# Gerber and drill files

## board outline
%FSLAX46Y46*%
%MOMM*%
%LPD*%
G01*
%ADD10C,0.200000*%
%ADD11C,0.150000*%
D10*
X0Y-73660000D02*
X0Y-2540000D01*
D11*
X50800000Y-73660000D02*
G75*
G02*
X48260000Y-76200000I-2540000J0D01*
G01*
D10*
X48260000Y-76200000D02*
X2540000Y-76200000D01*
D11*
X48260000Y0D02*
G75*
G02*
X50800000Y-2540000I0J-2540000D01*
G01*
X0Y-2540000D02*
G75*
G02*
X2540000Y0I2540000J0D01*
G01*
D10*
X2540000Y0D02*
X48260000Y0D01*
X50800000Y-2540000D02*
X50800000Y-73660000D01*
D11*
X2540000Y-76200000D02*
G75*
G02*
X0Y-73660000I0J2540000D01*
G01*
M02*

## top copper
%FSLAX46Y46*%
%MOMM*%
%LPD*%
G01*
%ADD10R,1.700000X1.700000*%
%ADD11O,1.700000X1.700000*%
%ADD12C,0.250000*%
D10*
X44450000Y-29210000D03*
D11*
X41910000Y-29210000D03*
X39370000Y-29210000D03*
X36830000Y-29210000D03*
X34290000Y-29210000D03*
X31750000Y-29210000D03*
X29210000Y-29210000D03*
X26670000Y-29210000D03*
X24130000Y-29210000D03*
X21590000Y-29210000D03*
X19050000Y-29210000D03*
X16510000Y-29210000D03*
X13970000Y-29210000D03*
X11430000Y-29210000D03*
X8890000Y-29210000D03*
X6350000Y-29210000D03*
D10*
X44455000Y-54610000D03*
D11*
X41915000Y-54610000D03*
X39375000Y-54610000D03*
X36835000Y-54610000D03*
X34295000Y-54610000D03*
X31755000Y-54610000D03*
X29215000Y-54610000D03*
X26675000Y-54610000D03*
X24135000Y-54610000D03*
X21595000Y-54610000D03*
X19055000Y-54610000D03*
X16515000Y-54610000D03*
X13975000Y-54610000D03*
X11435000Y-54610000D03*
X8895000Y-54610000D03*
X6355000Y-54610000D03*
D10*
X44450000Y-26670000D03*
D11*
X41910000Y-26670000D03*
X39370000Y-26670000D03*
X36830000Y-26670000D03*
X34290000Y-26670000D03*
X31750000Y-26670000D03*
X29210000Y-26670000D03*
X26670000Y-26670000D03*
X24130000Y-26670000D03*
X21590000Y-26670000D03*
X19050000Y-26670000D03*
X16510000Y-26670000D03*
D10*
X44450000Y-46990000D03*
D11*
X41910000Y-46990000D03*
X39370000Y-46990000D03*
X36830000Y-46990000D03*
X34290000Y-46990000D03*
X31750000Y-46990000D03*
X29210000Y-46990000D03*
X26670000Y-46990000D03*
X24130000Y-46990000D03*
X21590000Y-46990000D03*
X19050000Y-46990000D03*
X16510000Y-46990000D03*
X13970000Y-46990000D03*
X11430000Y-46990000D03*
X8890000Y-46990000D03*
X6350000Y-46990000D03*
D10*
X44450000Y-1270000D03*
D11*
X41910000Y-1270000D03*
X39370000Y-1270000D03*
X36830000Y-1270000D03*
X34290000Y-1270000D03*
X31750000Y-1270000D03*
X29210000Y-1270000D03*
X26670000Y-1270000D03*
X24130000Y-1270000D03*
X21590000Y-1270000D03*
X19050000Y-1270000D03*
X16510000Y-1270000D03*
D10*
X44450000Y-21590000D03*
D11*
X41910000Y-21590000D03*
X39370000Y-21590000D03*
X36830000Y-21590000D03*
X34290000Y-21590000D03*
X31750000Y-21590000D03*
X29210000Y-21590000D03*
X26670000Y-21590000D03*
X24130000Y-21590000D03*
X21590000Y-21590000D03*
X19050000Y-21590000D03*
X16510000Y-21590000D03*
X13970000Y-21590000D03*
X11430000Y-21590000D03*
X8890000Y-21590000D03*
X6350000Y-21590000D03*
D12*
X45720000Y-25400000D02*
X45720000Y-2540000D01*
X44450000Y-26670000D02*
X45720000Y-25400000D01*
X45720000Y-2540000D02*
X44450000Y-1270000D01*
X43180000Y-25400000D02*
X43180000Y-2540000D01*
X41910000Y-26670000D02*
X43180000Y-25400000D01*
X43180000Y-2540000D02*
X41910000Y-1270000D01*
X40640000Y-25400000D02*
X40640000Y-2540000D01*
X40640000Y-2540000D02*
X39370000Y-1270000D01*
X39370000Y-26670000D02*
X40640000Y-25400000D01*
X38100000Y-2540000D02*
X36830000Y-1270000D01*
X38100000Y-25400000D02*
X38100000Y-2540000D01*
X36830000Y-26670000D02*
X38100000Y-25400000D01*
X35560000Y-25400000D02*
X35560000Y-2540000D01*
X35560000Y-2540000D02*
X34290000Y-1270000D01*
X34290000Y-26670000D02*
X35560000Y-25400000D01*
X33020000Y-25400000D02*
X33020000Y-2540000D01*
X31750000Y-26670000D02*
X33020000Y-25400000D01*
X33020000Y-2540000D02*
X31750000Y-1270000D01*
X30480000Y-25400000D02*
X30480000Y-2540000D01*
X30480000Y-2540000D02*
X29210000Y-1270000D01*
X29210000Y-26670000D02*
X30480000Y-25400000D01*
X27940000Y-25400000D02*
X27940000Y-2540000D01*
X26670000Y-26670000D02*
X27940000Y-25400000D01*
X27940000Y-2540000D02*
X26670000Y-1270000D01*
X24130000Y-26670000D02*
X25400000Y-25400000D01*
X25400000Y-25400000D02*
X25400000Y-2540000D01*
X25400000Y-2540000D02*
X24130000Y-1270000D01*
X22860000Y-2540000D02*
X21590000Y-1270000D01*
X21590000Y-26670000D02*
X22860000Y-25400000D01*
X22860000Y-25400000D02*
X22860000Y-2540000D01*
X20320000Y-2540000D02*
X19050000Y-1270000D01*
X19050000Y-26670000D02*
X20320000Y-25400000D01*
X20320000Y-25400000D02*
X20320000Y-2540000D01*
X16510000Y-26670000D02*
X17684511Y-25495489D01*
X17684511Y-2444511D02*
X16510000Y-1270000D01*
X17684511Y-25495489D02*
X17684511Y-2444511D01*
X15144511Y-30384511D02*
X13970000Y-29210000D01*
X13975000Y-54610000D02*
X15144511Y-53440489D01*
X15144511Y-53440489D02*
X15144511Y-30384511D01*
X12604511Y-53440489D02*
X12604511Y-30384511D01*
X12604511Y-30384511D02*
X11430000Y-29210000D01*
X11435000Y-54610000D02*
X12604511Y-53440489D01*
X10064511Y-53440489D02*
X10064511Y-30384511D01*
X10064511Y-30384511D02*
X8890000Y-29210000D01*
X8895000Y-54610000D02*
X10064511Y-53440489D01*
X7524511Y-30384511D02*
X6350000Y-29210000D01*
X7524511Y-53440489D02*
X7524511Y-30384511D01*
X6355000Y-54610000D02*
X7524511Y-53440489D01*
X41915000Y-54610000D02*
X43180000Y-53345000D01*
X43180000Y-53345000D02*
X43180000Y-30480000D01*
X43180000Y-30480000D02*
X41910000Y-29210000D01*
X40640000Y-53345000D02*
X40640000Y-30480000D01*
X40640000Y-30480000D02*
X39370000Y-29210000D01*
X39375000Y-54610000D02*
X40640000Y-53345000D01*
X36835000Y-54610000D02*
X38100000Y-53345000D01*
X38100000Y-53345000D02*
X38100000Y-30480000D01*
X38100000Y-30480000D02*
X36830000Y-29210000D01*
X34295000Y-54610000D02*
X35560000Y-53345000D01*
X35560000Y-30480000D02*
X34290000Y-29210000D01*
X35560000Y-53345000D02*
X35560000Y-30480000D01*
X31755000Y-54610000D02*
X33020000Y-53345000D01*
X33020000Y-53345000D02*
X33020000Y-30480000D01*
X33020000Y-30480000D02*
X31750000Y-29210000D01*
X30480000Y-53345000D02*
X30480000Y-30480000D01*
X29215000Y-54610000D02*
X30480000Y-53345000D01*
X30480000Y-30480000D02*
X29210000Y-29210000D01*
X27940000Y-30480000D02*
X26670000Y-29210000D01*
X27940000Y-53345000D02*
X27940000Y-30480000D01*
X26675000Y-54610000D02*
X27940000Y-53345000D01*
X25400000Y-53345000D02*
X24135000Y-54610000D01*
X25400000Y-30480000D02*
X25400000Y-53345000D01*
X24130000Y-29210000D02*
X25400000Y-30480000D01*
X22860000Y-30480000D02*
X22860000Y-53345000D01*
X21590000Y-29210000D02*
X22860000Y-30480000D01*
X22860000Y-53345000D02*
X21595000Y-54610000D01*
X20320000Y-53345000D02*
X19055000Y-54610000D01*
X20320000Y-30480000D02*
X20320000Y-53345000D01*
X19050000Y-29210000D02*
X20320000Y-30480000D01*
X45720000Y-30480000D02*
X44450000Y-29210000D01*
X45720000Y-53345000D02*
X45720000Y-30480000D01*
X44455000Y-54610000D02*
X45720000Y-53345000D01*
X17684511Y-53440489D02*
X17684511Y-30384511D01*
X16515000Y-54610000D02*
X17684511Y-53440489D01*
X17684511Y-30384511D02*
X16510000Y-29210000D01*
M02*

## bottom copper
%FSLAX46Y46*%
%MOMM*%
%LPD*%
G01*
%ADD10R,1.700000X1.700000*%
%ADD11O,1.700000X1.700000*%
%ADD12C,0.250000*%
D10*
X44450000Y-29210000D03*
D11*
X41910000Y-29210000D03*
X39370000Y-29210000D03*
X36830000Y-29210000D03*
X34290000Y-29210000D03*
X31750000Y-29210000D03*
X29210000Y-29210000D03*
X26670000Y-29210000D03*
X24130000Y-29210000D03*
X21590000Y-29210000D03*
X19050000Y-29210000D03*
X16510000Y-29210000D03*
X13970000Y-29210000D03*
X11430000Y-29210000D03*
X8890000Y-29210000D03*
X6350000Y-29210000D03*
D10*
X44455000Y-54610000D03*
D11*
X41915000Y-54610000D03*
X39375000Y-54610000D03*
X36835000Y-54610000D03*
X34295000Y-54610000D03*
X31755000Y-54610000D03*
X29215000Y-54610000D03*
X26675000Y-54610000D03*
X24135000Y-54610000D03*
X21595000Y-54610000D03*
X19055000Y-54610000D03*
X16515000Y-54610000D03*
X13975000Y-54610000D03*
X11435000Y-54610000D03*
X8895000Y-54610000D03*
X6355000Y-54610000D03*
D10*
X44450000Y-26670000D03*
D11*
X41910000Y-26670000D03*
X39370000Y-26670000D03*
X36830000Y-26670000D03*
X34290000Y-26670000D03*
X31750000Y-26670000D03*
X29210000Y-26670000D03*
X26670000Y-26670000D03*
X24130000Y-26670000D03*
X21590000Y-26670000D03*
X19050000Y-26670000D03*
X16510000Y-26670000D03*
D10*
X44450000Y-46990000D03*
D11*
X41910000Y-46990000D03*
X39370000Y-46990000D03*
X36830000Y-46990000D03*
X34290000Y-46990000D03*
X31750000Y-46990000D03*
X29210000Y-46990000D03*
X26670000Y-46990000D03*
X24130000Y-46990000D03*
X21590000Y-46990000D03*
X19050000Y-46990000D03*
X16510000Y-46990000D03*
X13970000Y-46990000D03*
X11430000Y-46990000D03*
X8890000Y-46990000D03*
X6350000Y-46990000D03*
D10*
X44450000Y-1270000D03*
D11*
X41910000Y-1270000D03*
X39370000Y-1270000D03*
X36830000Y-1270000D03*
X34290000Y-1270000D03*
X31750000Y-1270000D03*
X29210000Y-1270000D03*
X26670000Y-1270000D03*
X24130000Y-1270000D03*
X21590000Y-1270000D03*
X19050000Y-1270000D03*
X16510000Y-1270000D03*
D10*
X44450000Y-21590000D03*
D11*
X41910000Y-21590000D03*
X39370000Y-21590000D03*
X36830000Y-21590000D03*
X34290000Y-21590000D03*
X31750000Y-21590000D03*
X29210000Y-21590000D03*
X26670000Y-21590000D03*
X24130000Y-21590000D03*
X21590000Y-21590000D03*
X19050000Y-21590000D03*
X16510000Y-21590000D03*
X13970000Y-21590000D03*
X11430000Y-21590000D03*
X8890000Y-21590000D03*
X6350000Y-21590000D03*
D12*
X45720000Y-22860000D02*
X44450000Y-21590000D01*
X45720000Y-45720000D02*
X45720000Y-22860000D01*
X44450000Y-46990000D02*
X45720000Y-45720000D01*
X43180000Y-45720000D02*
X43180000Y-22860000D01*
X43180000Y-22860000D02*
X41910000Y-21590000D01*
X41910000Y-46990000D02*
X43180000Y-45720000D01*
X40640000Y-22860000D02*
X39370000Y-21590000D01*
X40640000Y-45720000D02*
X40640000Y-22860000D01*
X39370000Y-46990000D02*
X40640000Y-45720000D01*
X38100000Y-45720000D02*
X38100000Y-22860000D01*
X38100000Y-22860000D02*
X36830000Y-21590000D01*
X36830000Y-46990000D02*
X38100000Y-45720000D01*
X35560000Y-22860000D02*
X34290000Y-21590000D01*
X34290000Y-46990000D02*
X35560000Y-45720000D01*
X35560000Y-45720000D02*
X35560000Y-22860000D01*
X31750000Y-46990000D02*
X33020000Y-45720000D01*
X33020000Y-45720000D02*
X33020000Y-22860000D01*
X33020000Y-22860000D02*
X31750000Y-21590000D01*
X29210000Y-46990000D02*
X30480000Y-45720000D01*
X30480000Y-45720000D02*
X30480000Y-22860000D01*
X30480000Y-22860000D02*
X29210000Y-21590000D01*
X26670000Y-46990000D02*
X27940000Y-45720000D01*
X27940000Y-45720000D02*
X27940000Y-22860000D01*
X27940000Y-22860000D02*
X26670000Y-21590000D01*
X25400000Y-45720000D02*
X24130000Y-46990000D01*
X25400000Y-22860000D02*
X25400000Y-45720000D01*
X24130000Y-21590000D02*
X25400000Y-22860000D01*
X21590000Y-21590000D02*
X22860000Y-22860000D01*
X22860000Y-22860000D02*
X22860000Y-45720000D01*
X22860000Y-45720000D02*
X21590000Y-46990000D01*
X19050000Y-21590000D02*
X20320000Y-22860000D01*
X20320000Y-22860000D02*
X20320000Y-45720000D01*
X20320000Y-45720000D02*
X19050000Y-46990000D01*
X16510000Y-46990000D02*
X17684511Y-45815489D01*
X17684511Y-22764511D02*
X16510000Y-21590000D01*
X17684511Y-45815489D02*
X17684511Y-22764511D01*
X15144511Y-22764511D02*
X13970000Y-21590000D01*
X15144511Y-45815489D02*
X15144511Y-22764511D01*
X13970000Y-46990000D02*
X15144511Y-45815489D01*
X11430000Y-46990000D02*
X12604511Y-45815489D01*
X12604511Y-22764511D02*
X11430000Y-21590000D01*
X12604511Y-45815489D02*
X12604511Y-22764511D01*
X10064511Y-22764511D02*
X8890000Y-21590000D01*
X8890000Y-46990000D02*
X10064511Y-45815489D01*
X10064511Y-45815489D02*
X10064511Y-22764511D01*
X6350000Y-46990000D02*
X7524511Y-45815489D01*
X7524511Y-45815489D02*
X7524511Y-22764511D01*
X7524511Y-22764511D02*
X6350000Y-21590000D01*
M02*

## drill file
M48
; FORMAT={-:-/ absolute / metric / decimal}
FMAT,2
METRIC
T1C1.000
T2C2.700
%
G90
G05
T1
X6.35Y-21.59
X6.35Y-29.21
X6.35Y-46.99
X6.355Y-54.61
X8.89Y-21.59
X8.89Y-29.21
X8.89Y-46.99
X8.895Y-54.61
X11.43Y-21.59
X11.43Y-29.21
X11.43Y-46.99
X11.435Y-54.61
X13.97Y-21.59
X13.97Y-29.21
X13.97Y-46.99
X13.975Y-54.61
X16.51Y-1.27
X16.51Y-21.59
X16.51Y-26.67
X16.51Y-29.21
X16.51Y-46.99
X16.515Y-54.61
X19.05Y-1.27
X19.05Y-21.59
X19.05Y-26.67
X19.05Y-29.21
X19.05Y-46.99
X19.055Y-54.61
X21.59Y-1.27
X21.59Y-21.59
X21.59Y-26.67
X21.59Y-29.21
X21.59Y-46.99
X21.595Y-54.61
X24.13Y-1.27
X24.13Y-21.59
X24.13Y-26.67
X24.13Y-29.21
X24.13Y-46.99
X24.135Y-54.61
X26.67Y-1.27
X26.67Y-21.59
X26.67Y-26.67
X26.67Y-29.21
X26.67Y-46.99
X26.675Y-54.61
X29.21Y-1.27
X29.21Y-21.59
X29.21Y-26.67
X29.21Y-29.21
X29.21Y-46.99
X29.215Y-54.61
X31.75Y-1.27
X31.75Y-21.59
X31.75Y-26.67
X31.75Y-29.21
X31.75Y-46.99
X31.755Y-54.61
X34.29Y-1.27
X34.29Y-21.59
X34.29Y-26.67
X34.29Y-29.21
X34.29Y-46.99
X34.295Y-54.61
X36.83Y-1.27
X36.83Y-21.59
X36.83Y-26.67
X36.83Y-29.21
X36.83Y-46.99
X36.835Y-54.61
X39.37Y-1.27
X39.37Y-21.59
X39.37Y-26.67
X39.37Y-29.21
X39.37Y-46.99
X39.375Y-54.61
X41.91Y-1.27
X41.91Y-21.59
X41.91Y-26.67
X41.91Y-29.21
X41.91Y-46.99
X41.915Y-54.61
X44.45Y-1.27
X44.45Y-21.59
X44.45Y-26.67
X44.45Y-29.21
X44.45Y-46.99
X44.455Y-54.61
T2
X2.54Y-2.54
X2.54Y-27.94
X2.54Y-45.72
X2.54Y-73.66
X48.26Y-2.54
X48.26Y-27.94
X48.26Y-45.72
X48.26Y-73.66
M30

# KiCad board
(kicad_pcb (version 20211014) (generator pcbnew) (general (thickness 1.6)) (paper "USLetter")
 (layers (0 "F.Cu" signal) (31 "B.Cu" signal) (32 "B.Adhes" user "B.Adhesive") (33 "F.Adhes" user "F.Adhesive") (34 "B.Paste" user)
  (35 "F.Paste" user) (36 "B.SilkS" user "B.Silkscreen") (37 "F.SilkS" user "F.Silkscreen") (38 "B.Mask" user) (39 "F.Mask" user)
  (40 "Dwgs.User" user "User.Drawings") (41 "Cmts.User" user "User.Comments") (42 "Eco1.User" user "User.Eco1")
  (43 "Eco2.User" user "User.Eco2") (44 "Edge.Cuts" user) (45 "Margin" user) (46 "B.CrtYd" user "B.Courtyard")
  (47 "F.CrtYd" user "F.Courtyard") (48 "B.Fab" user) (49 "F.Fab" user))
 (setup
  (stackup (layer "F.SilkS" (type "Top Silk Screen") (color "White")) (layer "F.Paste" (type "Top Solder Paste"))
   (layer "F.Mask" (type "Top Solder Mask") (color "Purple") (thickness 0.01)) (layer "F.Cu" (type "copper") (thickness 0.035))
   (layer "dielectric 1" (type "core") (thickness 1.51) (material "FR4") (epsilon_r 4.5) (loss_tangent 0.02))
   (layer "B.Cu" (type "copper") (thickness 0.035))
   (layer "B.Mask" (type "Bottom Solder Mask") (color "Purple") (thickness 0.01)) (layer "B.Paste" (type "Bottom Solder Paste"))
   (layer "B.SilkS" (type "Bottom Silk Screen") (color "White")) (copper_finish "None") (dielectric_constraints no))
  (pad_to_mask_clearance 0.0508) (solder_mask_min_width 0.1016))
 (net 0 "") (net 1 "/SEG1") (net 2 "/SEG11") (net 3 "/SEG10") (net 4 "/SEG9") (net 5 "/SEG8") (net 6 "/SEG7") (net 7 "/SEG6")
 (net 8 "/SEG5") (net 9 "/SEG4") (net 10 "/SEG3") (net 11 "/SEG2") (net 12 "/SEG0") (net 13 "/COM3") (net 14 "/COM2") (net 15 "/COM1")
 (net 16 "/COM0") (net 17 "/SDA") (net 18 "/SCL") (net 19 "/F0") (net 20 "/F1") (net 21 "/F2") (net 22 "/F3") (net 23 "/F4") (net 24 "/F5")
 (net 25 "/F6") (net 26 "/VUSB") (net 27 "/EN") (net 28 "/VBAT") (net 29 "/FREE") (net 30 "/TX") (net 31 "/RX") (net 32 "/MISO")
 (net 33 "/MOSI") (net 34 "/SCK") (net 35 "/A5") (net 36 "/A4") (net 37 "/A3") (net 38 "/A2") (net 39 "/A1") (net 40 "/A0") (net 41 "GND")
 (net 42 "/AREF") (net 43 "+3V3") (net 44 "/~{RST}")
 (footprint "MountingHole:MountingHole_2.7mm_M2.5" (layer "F.Cu") (at 48.26 2.54)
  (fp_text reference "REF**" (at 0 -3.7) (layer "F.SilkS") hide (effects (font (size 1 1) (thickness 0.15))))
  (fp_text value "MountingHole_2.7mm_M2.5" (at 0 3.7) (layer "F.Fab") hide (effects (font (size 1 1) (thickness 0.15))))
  (pad "" np_thru_hole circle locked (at 0 0) (size 2.7 2.7) (drill 2.7) (layers *.Cu *.Mask)))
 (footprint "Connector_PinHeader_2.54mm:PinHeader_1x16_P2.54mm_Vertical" (layer "F.Cu") (at 44.45 29.21 -90)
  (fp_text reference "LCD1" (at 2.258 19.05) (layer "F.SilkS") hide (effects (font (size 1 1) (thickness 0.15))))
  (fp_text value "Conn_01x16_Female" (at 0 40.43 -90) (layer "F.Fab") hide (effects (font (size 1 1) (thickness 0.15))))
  (pad "1" thru_hole rect (at 0 0 270) (size 1.7 1.7) (drill 1) (layers *.Cu *.Mask) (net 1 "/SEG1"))
  (pad "2" thru_hole oval (at 0 2.54 270) (size 1.7 1.7) (drill 1) (layers *.Cu *.Mask) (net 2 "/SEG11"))
  (pad "3" thru_hole oval (at 0 5.08 270) (size 1.7 1.7) (drill 1) (layers *.Cu *.Mask) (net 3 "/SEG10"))
  (pad "4" thru_hole oval (at 0 7.62 270) (size 1.7 1.7) (drill 1) (layers *.Cu *.Mask) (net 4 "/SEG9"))
  (pad "5" thru_hole oval (at 0 10.16 270) (size 1.7 1.7) (drill 1) (layers *.Cu *.Mask) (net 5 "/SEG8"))
  (pad "6" thru_hole oval (at 0 12.7 270) (size 1.7 1.7) (drill 1) (layers *.Cu *.Mask) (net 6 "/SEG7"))
  (pad "7" thru_hole oval (at 0 15.24 270) (size 1.7 1.7) (drill 1) (layers *.Cu *.Mask) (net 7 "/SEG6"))
  (pad "8" thru_hole oval (at 0 17.78 270) (size 1.7 1.7) (drill 1) (layers *.Cu *.Mask) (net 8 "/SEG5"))
  (pad "9" thru_hole oval (at 0 20.32 270) (size 1.7 1.7) (drill 1) (layers *.Cu *.Mask) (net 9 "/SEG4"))
  (pad "10" thru_hole oval (at 0 22.86 270) (size 1.7 1.7) (drill 1) (layers *.Cu *.Mask) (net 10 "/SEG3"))
  (pad "11" thru_hole oval (at 0 25.4 270) (size 1.7 1.7) (drill 1) (layers *.Cu *.Mask) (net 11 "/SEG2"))
  (pad "12" thru_hole oval (at 0 27.94 270) (size 1.7 1.7) (drill 1) (layers *.Cu *.Mask) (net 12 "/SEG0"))
  (pad "13" thru_hole oval (at 0 30.48 270) (size 1.7 1.7) (drill 1) (layers *.Cu *.Mask) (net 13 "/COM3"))
  (pad "14" thru_hole oval (at 0 33.02 270) (size 1.7 1.7) (drill 1) (layers *.Cu *.Mask) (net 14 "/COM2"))
  (pad "15" thru_hole oval (at 0 35.56 270) (size 1.7 1.7) (drill 1) (layers *.Cu *.Mask) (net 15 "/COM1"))
  (pad "16" thru_hole oval (at 0 38.1 270) (size 1.7 1.7) (drill 1) (layers *.Cu *.Mask) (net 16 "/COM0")))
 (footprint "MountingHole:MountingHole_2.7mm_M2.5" (layer "F.Cu") (at 2.54 27.94)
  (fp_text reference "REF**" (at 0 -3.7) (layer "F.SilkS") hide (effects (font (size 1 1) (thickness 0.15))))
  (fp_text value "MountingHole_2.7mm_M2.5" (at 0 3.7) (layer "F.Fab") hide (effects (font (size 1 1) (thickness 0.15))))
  (pad "" np_thru_hole circle locked (at 0 0) (size 2.7 2.7) (drill 2.7) (layers *.Cu *.Mask)))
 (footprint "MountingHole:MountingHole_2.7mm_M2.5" (layer "F.Cu") (at 2.54 73.66)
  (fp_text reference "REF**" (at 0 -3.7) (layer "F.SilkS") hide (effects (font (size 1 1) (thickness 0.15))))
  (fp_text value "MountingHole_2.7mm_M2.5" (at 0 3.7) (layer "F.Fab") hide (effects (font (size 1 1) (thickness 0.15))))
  (pad "" np_thru_hole circle locked (at 0 0) (size 2.7 2.7) (drill 2.7) (layers *.Cu *.Mask)))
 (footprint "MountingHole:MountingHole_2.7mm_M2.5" (layer "F.Cu") (at 2.54 45.72)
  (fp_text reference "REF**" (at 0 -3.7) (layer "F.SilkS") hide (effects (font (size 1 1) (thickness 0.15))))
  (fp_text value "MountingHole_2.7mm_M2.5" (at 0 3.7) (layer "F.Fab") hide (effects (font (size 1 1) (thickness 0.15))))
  (pad "" np_thru_hole circle locked (at 0 0) (size 2.7 2.7) (drill 2.7) (layers *.Cu *.Mask)))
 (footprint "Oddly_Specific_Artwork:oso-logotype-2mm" (layer "F.Cu") (at 25.4 70.866)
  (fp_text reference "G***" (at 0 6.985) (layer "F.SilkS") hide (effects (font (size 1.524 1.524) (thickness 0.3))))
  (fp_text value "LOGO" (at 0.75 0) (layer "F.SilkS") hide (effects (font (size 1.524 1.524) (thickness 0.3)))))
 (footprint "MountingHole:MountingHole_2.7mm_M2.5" (layer "F.Cu") (at 48.26 45.72)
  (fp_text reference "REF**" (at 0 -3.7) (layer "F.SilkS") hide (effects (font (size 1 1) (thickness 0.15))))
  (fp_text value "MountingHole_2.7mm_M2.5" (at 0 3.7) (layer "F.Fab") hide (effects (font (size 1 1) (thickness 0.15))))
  (pad "" np_thru_hole circle locked (at 0 0) (size 2.7 2.7) (drill 2.7) (layers *.Cu *.Mask)))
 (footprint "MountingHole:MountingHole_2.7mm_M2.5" (layer "F.Cu") (at 48.26 73.66)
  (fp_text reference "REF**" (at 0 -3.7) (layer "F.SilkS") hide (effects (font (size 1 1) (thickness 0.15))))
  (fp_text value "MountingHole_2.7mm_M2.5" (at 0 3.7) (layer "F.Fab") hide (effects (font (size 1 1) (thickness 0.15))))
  (pad "" np_thru_hole circle locked (at 0 0) (size 2.7 2.7) (drill 2.7) (layers *.Cu *.Mask)))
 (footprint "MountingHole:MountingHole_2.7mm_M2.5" (layer "F.Cu") (at 2.54 2.54)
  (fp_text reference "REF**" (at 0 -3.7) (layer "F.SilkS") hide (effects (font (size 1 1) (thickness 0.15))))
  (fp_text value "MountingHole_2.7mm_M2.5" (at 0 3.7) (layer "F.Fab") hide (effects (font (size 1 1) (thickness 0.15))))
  (pad "" np_thru_hole circle locked (at 0 0) (size 2.7 2.7) (drill 2.7) (layers *.Cu *.Mask)))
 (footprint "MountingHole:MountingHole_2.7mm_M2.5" (layer "F.Cu") (at 48.26 27.94)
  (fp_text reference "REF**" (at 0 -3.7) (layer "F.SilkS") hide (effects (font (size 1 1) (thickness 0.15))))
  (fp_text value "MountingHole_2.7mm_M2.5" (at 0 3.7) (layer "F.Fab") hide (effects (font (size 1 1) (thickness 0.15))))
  (pad "" np_thru_hole circle locked (at 0 0) (size 2.7 2.7) (drill 2.7) (layers *.Cu *.Mask)))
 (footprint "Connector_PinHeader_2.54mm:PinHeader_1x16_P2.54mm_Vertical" (layer "F.Cu") (at 44.455 54.61 -90)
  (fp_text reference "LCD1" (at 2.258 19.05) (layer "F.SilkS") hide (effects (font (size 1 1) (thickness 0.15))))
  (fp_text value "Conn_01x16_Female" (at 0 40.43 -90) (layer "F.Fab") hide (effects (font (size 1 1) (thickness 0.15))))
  (pad "1" thru_hole rect (at 0 0 270) (size 1.7 1.7) (drill 1) (layers *.Cu *.Mask) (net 1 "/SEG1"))
  (pad "2" thru_hole oval (at 0 2.54 270) (size 1.7 1.7) (drill 1) (layers *.Cu *.Mask) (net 2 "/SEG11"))
  (pad "3" thru_hole oval (at 0 5.08 270) (size 1.7 1.7) (drill 1) (layers *.Cu *.Mask) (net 3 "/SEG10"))
  (pad "4" thru_hole oval (at 0 7.62 270) (size 1.7 1.7) (drill 1) (layers *.Cu *.Mask) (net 4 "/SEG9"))
  (pad "5" thru_hole oval (at 0 10.16 270) (size 1.7 1.7) (drill 1) (layers *.Cu *.Mask) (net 5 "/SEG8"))
  (pad "6" thru_hole oval (at 0 12.7 270) (size 1.7 1.7) (drill 1) (layers *.Cu *.Mask) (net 6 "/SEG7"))
  (pad "7" thru_hole oval (at 0 15.24 270) (size 1.7 1.7) (drill 1) (layers *.Cu *.Mask) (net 7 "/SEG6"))
  (pad "8" thru_hole oval (at 0 17.78 270) (size 1.7 1.7) (drill 1) (layers *.Cu *.Mask) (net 8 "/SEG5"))
  (pad "9" thru_hole oval (at 0 20.32 270) (size 1.7 1.7) (drill 1) (layers *.Cu *.Mask) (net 9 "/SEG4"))
  (pad "10" thru_hole oval (at 0 22.86 270) (size 1.7 1.7) (drill 1) (layers *.Cu *.Mask) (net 10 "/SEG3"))
  (pad "11" thru_hole oval (at 0 25.4 270) (size 1.7 1.7) (drill 1) (layers *.Cu *.Mask) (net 11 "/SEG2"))
  (pad "12" thru_hole oval (at 0 27.94 270) (size 1.7 1.7) (drill 1) (layers *.Cu *.Mask) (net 12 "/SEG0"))
  (pad "13" thru_hole oval (at 0 30.48 270) (size 1.7 1.7) (drill 1) (layers *.Cu *.Mask) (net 13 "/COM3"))
  (pad "14" thru_hole oval (at 0 33.02 270) (size 1.7 1.7) (drill 1) (layers *.Cu *.Mask) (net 14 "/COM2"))
  (pad "15" thru_hole oval (at 0 35.56 270) (size 1.7 1.7) (drill 1) (layers *.Cu *.Mask) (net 15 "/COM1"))
  (pad "16" thru_hole oval (at 0 38.1 270) (size 1.7 1.7) (drill 1) (layers *.Cu *.Mask) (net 16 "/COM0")))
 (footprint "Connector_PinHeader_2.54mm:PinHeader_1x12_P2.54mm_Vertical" (layer "B.Cu") (at 44.45 26.67 90)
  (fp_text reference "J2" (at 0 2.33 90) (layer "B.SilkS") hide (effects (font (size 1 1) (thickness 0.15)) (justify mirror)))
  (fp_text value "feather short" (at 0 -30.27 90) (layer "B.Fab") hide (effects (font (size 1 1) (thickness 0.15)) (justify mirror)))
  (pad "1" thru_hole rect locked (at 0 0 90) (size 1.7 1.7) (drill 1) (layers *.Cu *.Mask) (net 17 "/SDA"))
  (pad "2" thru_hole oval locked (at 0 -2.54 90) (size 1.7 1.7) (drill 1) (layers *.Cu *.Mask) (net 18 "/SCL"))
  (pad "3" thru_hole oval locked (at 0 -5.08 90) (size 1.7 1.7) (drill 1) (layers *.Cu *.Mask) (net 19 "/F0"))
  (pad "4" thru_hole oval locked (at 0 -7.62 90) (size 1.7 1.7) (drill 1) (layers *.Cu *.Mask) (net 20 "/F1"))
  (pad "5" thru_hole oval locked (at 0 -10.16 90) (size 1.7 1.7) (drill 1) (layers *.Cu *.Mask) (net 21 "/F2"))
  (pad "6" thru_hole oval locked (at 0 -12.7 90) (size 1.7 1.7) (drill 1) (layers *.Cu *.Mask) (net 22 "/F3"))
  (pad "7" thru_hole oval locked (at 0 -15.24 90) (size 1.7 1.7) (drill 1) (layers *.Cu *.Mask) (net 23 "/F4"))
  (pad "8" thru_hole oval locked (at 0 -17.78 90) (size 1.7 1.7) (drill 1) (layers *.Cu *.Mask) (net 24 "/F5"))
  (pad "9" thru_hole oval locked (at 0 -20.32 90) (size 1.7 1.7) (drill 1) (layers *.Cu *.Mask) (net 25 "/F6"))
  (pad "10" thru_hole oval locked (at 0 -22.86 90) (size 1.7 1.7) (drill 1) (layers *.Cu *.Mask) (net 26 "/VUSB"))
  (pad "11" thru_hole oval locked (at 0 -25.4 90) (size 1.7 1.7) (drill 1) (layers *.Cu *.Mask) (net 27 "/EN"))
  (pad "12" thru_hole oval locked (at 0 -27.94 90) (size 1.7 1.7) (drill 1) (layers *.Cu *.Mask) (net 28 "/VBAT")))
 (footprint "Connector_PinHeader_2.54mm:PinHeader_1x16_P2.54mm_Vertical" (layer "B.Cu") (at 44.45 46.99 90)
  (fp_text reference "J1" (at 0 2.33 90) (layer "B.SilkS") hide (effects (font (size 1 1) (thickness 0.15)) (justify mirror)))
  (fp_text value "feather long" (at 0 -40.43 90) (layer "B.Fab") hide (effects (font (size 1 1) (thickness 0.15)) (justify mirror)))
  (pad "1" thru_hole rect locked (at 0 0 90) (size 1.7 1.7) (drill 1) (layers *.Cu *.Mask) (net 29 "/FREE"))
  (pad "2" thru_hole oval locked (at 0 -2.54 90) (size 1.7 1.7) (drill 1) (layers *.Cu *.Mask) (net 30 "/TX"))
  (pad "3" thru_hole oval locked (at 0 -5.08 90) (size 1.7 1.7) (drill 1) (layers *.Cu *.Mask) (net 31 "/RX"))
  (pad "4" thru_hole oval locked (at 0 -7.62 90) (size 1.7 1.7) (drill 1) (layers *.Cu *.Mask) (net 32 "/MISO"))
  (pad "5" thru_hole oval locked (at 0 -10.16 90) (size 1.7 1.7) (drill 1) (layers *.Cu *.Mask) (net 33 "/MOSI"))
  (pad "6" thru_hole oval locked (at 0 -12.7 90) (size 1.7 1.7) (drill 1) (layers *.Cu *.Mask) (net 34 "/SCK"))
  (pad "7" thru_hole oval locked (at 0 -15.24 90) (size 1.7 1.7) (drill 1) (layers *.Cu *.Mask) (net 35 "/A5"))
  (pad "8" thru_hole oval locked (at 0 -17.78 90) (size 1.7 1.7) (drill 1) (layers *.Cu *.Mask) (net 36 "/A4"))
  (pad "9" thru_hole oval locked (at 0 -20.32 90) (size 1.7 1.7) (drill 1) (layers *.Cu *.Mask) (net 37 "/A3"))
  (pad "10" thru_hole oval locked (at 0 -22.86 90) (size 1.7 1.7) (drill 1) (layers *.Cu *.Mask) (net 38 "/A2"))
  (pad "11" thru_hole oval locked (at 0 -25.4 90) (size 1.7 1.7) (drill 1) (layers *.Cu *.Mask) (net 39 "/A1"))
  (pad "12" thru_hole oval locked (at 0 -27.94 90) (size 1.7 1.7) (drill 1) (layers *.Cu *.Mask) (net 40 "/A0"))
  (pad "13" thru_hole oval locked (at 0 -30.48 90) (size 1.7 1.7) (drill 1) (layers *.Cu *.Mask) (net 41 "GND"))
  (pad "14" thru_hole oval locked (at 0 -33.02 90) (size 1.7 1.7) (drill 1) (layers *.Cu *.Mask) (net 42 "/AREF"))
  (pad "15" thru_hole oval locked (at 0 -35.56 90) (size 1.7 1.7) (drill 1) (layers *.Cu *.Mask) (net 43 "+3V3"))
  (pad "16" thru_hole oval locked (at 0 -38.1 90) (size 1.7 1.7) (drill 1) (layers *.Cu *.Mask) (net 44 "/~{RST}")))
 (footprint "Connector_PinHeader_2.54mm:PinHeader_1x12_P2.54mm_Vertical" (layer "B.Cu") (at 44.45 1.27 90)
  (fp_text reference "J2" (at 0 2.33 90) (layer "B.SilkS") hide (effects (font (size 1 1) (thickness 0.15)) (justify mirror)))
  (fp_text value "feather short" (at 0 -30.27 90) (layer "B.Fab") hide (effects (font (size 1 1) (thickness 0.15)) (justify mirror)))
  (pad "1" thru_hole rect locked (at 0 0 90) (size 1.7 1.7) (drill 1) (layers *.Cu *.Mask) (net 17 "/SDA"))
  (pad "2" thru_hole oval locked (at 0 -2.54 90) (size 1.7 1.7) (drill 1) (layers *.Cu *.Mask) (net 18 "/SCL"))
  (pad "3" thru_hole oval locked (at 0 -5.08 90) (size 1.7 1.7) (drill 1) (layers *.Cu *.Mask) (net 19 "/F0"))
  (pad "4" thru_hole oval locked (at 0 -7.62 90) (size 1.7 1.7) (drill 1) (layers *.Cu *.Mask) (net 20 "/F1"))
  (pad "5" thru_hole oval locked (at 0 -10.16 90) (size 1.7 1.7) (drill 1) (layers *.Cu *.Mask) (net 21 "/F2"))
  (pad "6" thru_hole oval locked (at 0 -12.7 90) (size 1.7 1.7) (drill 1) (layers *.Cu *.Mask) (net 22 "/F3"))
  (pad "7" thru_hole oval locked (at 0 -15.24 90) (size 1.7 1.7) (drill 1) (layers *.Cu *.Mask) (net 23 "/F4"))
  (pad "8" thru_hole oval locked (at 0 -17.78 90) (size 1.7 1.7) (drill 1) (layers *.Cu *.Mask) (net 24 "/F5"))
  (pad "9" thru_hole oval locked (at 0 -20.32 90) (size 1.7 1.7) (drill 1) (layers *.Cu *.Mask) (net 25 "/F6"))
  (pad "10" thru_hole oval locked (at 0 -22.86 90) (size 1.7 1.7) (drill 1) (layers *.Cu *.Mask) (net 26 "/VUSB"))
  (pad "11" thru_hole oval locked (at 0 -25.4 90) (size 1.7 1.7) (drill 1) (layers *.Cu *.Mask) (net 27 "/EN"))
  (pad "12" thru_hole oval locked (at 0 -27.94 90) (size 1.7 1.7) (drill 1) (layers *.Cu *.Mask) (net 28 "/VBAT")))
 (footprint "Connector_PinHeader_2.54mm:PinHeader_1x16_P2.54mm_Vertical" (layer "B.Cu") (at 44.45 21.59 90)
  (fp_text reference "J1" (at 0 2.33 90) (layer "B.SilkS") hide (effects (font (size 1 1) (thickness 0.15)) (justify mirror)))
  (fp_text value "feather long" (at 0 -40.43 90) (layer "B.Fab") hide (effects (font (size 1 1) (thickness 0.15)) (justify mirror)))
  (pad "1" thru_hole rect locked (at 0 0 90) (size 1.7 1.7) (drill 1) (layers *.Cu *.Mask) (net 29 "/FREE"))
  (pad "2" thru_hole oval locked (at 0 -2.54 90) (size 1.7 1.7) (drill 1) (layers *.Cu *.Mask) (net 30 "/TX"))
  (pad "3" thru_hole oval locked (at 0 -5.08 90) (size 1.7 1.7) (drill 1) (layers *.Cu *.Mask) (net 31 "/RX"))
  (pad "4" thru_hole oval locked (at 0 -7.62 90) (size 1.7 1.7) (drill 1) (layers *.Cu *.Mask) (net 32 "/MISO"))
  (pad "5" thru_hole oval locked (at 0 -10.16 90) (size 1.7 1.7) (drill 1) (layers *.Cu *.Mask) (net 33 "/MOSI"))
  (pad "6" thru_hole oval locked (at 0 -12.7 90) (size 1.7 1.7) (drill 1) (layers *.Cu *.Mask) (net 34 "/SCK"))
  (pad "7" thru_hole oval locked (at 0 -15.24 90) (size 1.7 1.7) (drill 1) (layers *.Cu *.Mask) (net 35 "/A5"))
  (pad "8" thru_hole oval locked (at 0 -17.78 90) (size 1.7 1.7) (drill 1) (layers *.Cu *.Mask) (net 36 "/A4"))
  (pad "9" thru_hole oval locked (at 0 -20.32 90) (size 1.7 1.7) (drill 1) (layers *.Cu *.Mask) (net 37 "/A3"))
  (pad "10" thru_hole oval locked (at 0 -22.86 90) (size 1.7 1.7) (drill 1) (layers *.Cu *.Mask) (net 38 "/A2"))
  (pad "11" thru_hole oval locked (at 0 -25.4 90) (size 1.7 1.7) (drill 1) (layers *.Cu *.Mask) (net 39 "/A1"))
  (pad "12" thru_hole oval locked (at 0 -27.94 90) (size 1.7 1.7) (drill 1) (layers *.Cu *.Mask) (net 40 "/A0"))
  (pad "13" thru_hole oval locked (at 0 -30.48 90) (size 1.7 1.7) (drill 1) (layers *.Cu *.Mask) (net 41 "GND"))
  (pad "14" thru_hole oval locked (at 0 -33.02 90) (size 1.7 1.7) (drill 1) (layers *.Cu *.Mask) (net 42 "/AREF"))
  (pad "15" thru_hole oval locked (at 0 -35.56 90) (size 1.7 1.7) (drill 1) (layers *.Cu *.Mask) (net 43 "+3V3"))
  (pad "16" thru_hole oval locked (at 0 -38.1 90) (size 1.7 1.7) (drill 1) (layers *.Cu *.Mask) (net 44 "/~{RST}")))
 (gr_line (start 0 73.66) (end 0 2.54) (layer "Edge.Cuts") (width 0.2))
 (gr_arc (start 50.8 73.66) (mid 50.056051 75.456051) (end 48.26 76.2) (layer "Edge.Cuts") (width 0.15))
 (gr_line (start 48.26 76.2) (end 2.54 76.2) (layer "Edge.Cuts") (width 0.2))
 (gr_arc (start 48.26 0) (mid 50.056051 0.743949) (end 50.8 2.54) (layer "Edge.Cuts") (width 0.15))
 (gr_arc (start 0 2.54) (mid 0.743949 0.743949) (end 2.54 0) (layer "Edge.Cuts") (width 0.15))
 (gr_line (start 2.54 0) (end 48.26 0) (layer "Edge.Cuts") (width 0.2))
 (gr_line (start 50.8 2.54) (end 50.8 73.66) (layer "Edge.Cuts") (width 0.2))
 (gr_arc (start 2.54 76.2) (mid 0.743949 75.456051) (end 0 73.66) (layer "Edge.Cuts") (width 0.15))
 (segment (start 45.72 22.86) (end 44.45 21.59) (width 0.25) (layer "B.Cu") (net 29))
 (segment (start 45.72 45.72) (end 45.72 22.86) (width 0.25) (layer "B.Cu") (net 29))
 (segment (start 44.45 46.99) (end 45.72 45.72) (width 0.25) (layer "B.Cu") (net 29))
 (segment (start 43.18 45.72) (end 43.18 22.86) (width 0.25) (layer "B.Cu") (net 30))
 (segment (start 43.18 22.86) (end 41.91 21.59) (width 0.25) (layer "B.Cu") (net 30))
 (segment (start 41.91 46.99) (end 43.18 45.72) (width 0.25) (layer "B.Cu") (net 30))
 (segment (start 40.64 22.86) (end 39.37 21.59) (width 0.25) (layer "B.Cu") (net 31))
 (segment (start 40.64 45.72) (end 40.64 22.86) (width 0.25) (layer "B.Cu") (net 31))
 (segment (start 39.37 46.99) (end 40.64 45.72) (width 0.25) (layer "B.Cu") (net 31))
 (segment (start 38.1 45.72) (end 38.1 22.86) (width 0.25) (layer "B.Cu") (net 32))
 (segment (start 38.1 22.86) (end 36.83 21.59) (width 0.25) (layer "B.Cu") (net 32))
 (segment (start 36.83 46.99) (end 38.1 45.72) (width 0.25) (layer "B.Cu") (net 32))
 (segment (start 35.56 22.86) (end 34.29 21.59) (width 0.25) (layer "B.Cu") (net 33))
 (segment (start 34.29 46.99) (end 35.56 45.72) (width 0.25) (layer "B.Cu") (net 33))
 (segment (start 35.56 45.72) (end 35.56 22.86) (width 0.25) (layer "B.Cu") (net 33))
 (segment (start 31.75 46.99) (end 33.02 45.72) (width 0.25) (layer "B.Cu") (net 34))
 (segment (start 33.02 45.72) (end 33.02 22.86) (width 0.25) (layer "B.Cu") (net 34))
 (segment (start 33.02 22.86) (end 31.75 21.59) (width 0.25) (layer "B.Cu") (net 34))
 (segment (start 29.21 46.99) (end 30.48 45.72) (width 0.25) (layer "B.Cu") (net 35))
 (segment (start 30.48 45.72) (end 30.48 22.86) (width 0.25) (layer "B.Cu") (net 35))
 (segment (start 30.48 22.86) (end 29.21 21.59) (width 0.25) (layer "B.Cu") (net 35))
 (segment (start 26.67 46.99) (end 27.94 45.72) (width 0.25) (layer "B.Cu") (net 36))
 (segment (start 27.94 45.72) (end 27.94 22.86) (width 0.25) (layer "B.Cu") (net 36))
 (segment (start 27.94 22.86) (end 26.67 21.59) (width 0.25) (layer "B.Cu") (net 36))
 (segment (start 25.4 45.72) (end 24.13 46.99) (width 0.25) (layer "B.Cu") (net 37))
 (segment (start 25.4 22.86) (end 25.4 45.72) (width 0.25) (layer "B.Cu") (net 37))
 (segment (start 24.13 21.59) (end 25.4 22.86) (width 0.25) (layer "B.Cu") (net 37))
 (segment (start 21.59 21.59) (end 22.86 22.86) (width 0.25) (layer "B.Cu") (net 38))
 (segment (start 22.86 22.86) (end 22.86 45.72) (width 0.25) (layer "B.Cu") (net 38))
 (segment (start 22.86 45.72) (end 21.59 46.99) (width 0.25) (layer "B.Cu") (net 38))
 (segment (start 19.05 21.59) (end 20.32 22.86) (width 0.25) (layer "B.Cu") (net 39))
 (segment (start 20.32 22.86) (end 20.32 45.72) (width 0.25) (layer "B.Cu") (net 39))
 (segment (start 20.32 45.72) (end 19.05 46.99) (width 0.25) (layer "B.Cu") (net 39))
 (segment (start 16.51 46.99) (end 17.684511 45.815489) (width 0.25) (layer "B.Cu") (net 40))
 (segment (start 17.684511 22.764511) (end 16.51 21.59) (width 0.25) (layer "B.Cu") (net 40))
 (segment (start 17.684511 45.815489) (end 17.684511 22.764511) (width 0.25) (layer "B.Cu") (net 40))
 (segment (start 15.144511 22.764511) (end 13.97 21.59) (width 0.25) (layer "B.Cu") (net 41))
 (segment (start 15.144511 45.815489) (end 15.144511 22.764511) (width 0.25) (layer "B.Cu") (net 41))
 (segment (start 13.97 46.99) (end 15.144511 45.815489) (width 0.25) (layer "B.Cu") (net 41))
 (segment (start 11.43 46.99) (end 12.604511 45.815489) (width 0.25) (layer "B.Cu") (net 42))
 (segment (start 12.604511 22.764511) (end 11.43 21.59) (width 0.25) (layer "B.Cu") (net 42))
 (segment (start 12.604511 45.815489) (end 12.604511 22.764511) (width 0.25) (layer "B.Cu") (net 42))
 (segment (start 10.064511 22.764511) (end 8.89 21.59) (width 0.25) (layer "B.Cu") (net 43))
 (segment (start 8.89 46.99) (end 10.064511 45.815489) (width 0.25) (layer "B.Cu") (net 43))
 (segment (start 10.064511 45.815489) (end 10.064511 22.764511) (width 0.25) (layer "B.Cu") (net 43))
 (segment (start 6.35 46.99) (end 7.524511 45.815489) (width 0.25) (layer "B.Cu") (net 44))
 (segment (start 7.524511 45.815489) (end 7.524511 22.764511) (width 0.25) (layer "B.Cu") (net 44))
 (segment (start 7.524511 22.764511) (end 6.35 21.59) (width 0.25) (layer "B.Cu") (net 44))
 (segment (start 45.72 25.4) (end 45.72 2.54) (width 0.25) (layer "F.Cu") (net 17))
 (segment (start 44.45 26.67) (end 45.72 25.4) (width 0.25) (layer "F.Cu") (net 17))
 (segment (start 45.72 2.54) (end 44.45 1.27) (width 0.25) (layer "F.Cu") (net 17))
 (segment (start 43.18 25.4) (end 43.18 2.54) (width 0.25) (layer "F.Cu") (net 18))
 (segment (start 41.91 26.67) (end 43.18 25.4) (width 0.25) (layer "F.Cu") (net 18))
 (segment (start 43.18 2.54) (end 41.91 1.27) (width 0.25) (layer "F.Cu") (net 18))
 (segment (start 40.64 25.4) (end 40.64 2.54) (width 0.25) (layer "F.Cu") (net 19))
 (segment (start 40.64 2.54) (end 39.37 1.27) (width 0.25) (layer "F.Cu") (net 19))
 (segment (start 39.37 26.67) (end 40.64 25.4) (width 0.25) (layer "F.Cu") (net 19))
 (segment (start 38.1 2.54) (end 36.83 1.27) (width 0.25) (layer "F.Cu") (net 20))
 (segment (start 38.1 25.4) (end 38.1 2.54) (width 0.25) (layer "F.Cu") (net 20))
 (segment (start 36.83 26.67) (end 38.1 25.4) (width 0.25) (layer "F.Cu") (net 20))
 (segment (start 35.56 25.4) (end 35.56 2.54) (width 0.25) (layer "F.Cu") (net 21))
 (segment (start 35.56 2.54) (end 34.29 1.27) (width 0.25) (layer "F.Cu") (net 21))
 (segment (start 34.29 26.67) (end 35.56 25.4) (width 0.25) (layer "F.Cu") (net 21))
 (segment (start 33.02 25.4) (end 33.02 2.54) (width 0.25) (layer "F.Cu") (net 22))
 (segment (start 31.75 26.67) (end 33.02 25.4) (width 0.25) (layer "F.Cu") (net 22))
 (segment (start 33.02 2.54) (end 31.75 1.27) (width 0.25) (layer "F.Cu") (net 22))
 (segment (start 30.48 25.4) (end 30.48 2.54) (width 0.25) (layer "F.Cu") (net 23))
 (segment (start 30.48 2.54) (end 29.21 1.27) (width 0.25) (layer "F.Cu") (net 23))
 (segment (start 29.21 26.67) (end 30.48 25.4) (width 0.25) (layer "F.Cu") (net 23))
 (segment (start 27.94 25.4) (end 27.94 2.54) (width 0.25) (layer "F.Cu") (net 24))
 (segment (start 26.67 26.67) (end 27.94 25.4) (width 0.25) (layer "F.Cu") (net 24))
 (segment (start 27.94 2.54) (end 26.67 1.27) (width 0.25) (layer "F.Cu") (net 24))
 (segment (start 24.13 26.67) (end 25.4 25.4) (width 0.25) (layer "F.Cu") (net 25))
 (segment (start 25.4 25.4) (end 25.4 2.54) (width 0.25) (layer "F.Cu") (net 25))
 (segment (start 25.4 2.54) (end 24.13 1.27) (width 0.25) (layer "F.Cu") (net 25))
 (segment (start 22.86 2.54) (end 21.59 1.27) (width 0.25) (layer "F.Cu") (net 26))
 (segment (start 21.59 26.67) (end 22.86 25.4) (width 0.25) (layer "F.Cu") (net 26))
 (segment (start 22.86 25.4) (end 22.86 2.54) (width 0.25) (layer "F.Cu") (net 26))
 (segment (start 20.32 2.54) (end 19.05 1.27) (width 0.25) (layer "F.Cu") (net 27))
 (segment (start 19.05 26.67) (end 20.32 25.4) (width 0.25) (layer "F.Cu") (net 27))
 (segment (start 20.32 25.4) (end 20.32 2.54) (width 0.25) (layer "F.Cu") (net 27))
 (segment (start 16.51 26.67) (end 17.684511 25.495489) (width 0.25) (layer "F.Cu") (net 28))
 (segment (start 17.684511 2.444511) (end 16.51 1.27) (width 0.25) (layer "F.Cu") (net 28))
 (segment (start 17.684511 25.495489) (end 17.684511 2.444511) (width 0.25) (layer "F.Cu") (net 28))
 (segment (start 15.144511 30.384511) (end 13.97 29.21) (width 0.25) (layer "F.Cu") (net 13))
 (segment (start 13.975 54.61) (end 15.144511 53.440489) (width 0.25) (layer "F.Cu") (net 13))
 (segment (start 15.144511 53.440489) (end 15.144511 30.384511) (width 0.25) (layer "F.Cu") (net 13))
 (segment (start 12.604511 53.440489) (end 12.604511 30.384511) (width 0.25) (layer "F.Cu") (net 14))
 (segment (start 12.604511 30.384511) (end 11.43 29.21) (width 0.25) (layer "F.Cu") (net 14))
 (segment (start 11.435 54.61) (end 12.604511 53.440489) (width 0.25) (layer "F.Cu") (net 14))
 (segment (start 10.064511 53.440489) (end 10.064511 30.384511) (width 0.25) (layer "F.Cu") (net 15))
 (segment (start 10.064511 30.384511) (end 8.89 29.21) (width 0.25) (layer "F.Cu") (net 15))
 (segment (start 8.895 54.61) (end 10.064511 53.440489) (width 0.25) (layer "F.Cu") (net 15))
 (segment (start 7.524511 30.384511) (end 6.35 29.21) (width 0.25) (layer "F.Cu") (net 16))
 (segment (start 7.524511 53.440489) (end 7.524511 30.384511) (width 0.25) (layer "F.Cu") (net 16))
 (segment (start 6.355 54.61) (end 7.524511 53.440489) (width 0.25) (layer "F.Cu") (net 16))
 (segment (start 41.915 54.61) (end 43.18 53.345) (width 0.25) (layer "F.Cu") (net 2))
 (segment (start 43.18 53.345) (end 43.18 30.48) (width 0.25) (layer "F.Cu") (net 2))
 (segment (start 43.18 30.48) (end 41.91 29.21) (width 0.25) (layer "F.Cu") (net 2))
 (segment (start 40.64 53.345) (end 40.64 30.48) (width 0.25) (layer "F.Cu") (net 3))
 (segment (start 40.64 30.48) (end 39.37 29.21) (width 0.25) (layer "F.Cu") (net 3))
 (segment (start 39.375 54.61) (end 40.64 53.345) (width 0.25) (layer "F.Cu") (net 3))
 (segment (start 36.835 54.61) (end 38.1 53.345) (width 0.25) (layer "F.Cu") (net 4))
 (segment (start 38.1 53.345) (end 38.1 30.48) (width 0.25) (layer "F.Cu") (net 4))
 (segment (start 38.1 30.48) (end 36.83 29.21) (width 0.25) (layer "F.Cu") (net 4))
 (segment (start 34.295 54.61) (end 35.56 53.345) (width 0.25) (layer "F.Cu") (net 5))
 (segment (start 35.56 30.48) (end 34.29 29.21) (width 0.25) (layer "F.Cu") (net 5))
 (segment (start 35.56 53.345) (end 35.56 30.48) (width 0.25) (layer "F.Cu") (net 5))
 (segment (start 31.755 54.61) (end 33.02 53.345) (width 0.25) (layer "F.Cu") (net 6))
 (segment (start 33.02 53.345) (end 33.02 30.48) (width 0.25) (layer "F.Cu") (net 6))
 (segment (start 33.02 30.48) (end 31.75 29.21) (width 0.25) (layer "F.Cu") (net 6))
 (segment (start 30.48 53.345) (end 30.48 30.48) (width 0.25) (layer "F.Cu") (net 7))
 (segment (start 29.215 54.61) (end 30.48 53.345) (width 0.25) (layer "F.Cu") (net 7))
 (segment (start 30.48 30.48) (end 29.21 29.21) (width 0.25) (layer "F.Cu") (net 7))
 (segment (start 27.94 30.48) (end 26.67 29.21) (width 0.25) (layer "F.Cu") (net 8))
 (segment (start 27.94 53.345) (end 27.94 30.48) (width 0.25) (layer "F.Cu") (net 8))
 (segment (start 26.675 54.61) (end 27.94 53.345) (width 0.25) (layer "F.Cu") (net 8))
 (segment (start 25.4 53.345) (end 24.135 54.61) (width 0.25) (layer "F.Cu") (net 9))
 (segment (start 25.4 30.48) (end 25.4 53.345) (width 0.25) (layer "F.Cu") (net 9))
 (segment (start 24.13 29.21) (end 25.4 30.48) (width 0.25) (layer "F.Cu") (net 9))
 (segment (start 22.86 30.48) (end 22.86 53.345) (width 0.25) (layer "F.Cu") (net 10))
 (segment (start 21.59 29.21) (end 22.86 30.48) (width 0.25) (layer "F.Cu") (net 10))
 (segment (start 22.86 53.345) (end 21.595 54.61) (width 0.25) (layer "F.Cu") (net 10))
 (segment (start 20.32 53.345) (end 19.055 54.61) (width 0.25) (layer "F.Cu") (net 11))
 (segment (start 20.32 30.48) (end 20.32 53.345) (width 0.25) (layer "F.Cu") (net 11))
 (segment (start 19.05 29.21) (end 20.32 30.48) (width 0.25) (layer "F.Cu") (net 11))
 (segment (start 45.72 30.48) (end 44.45 29.21) (width 0.25) (layer "F.Cu") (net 1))
 (segment (start 45.72 53.345) (end 45.72 30.48) (width 0.25) (layer "F.Cu") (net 1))
 (segment (start 44.455 54.61) (end 45.72 53.345) (width 0.25) (layer "F.Cu") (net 1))
 (segment (start 17.684511 53.440489) (end 17.684511 30.384511) (width 0.25) (layer "F.Cu") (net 12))
 (segment (start 16.515 54.61) (end 17.684511 53.440489) (width 0.25) (layer "F.Cu") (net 12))
 (segment (start 17.684511 30.384511) (end 16.51 29.21) (width 0.25) (layer "F.Cu") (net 12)))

